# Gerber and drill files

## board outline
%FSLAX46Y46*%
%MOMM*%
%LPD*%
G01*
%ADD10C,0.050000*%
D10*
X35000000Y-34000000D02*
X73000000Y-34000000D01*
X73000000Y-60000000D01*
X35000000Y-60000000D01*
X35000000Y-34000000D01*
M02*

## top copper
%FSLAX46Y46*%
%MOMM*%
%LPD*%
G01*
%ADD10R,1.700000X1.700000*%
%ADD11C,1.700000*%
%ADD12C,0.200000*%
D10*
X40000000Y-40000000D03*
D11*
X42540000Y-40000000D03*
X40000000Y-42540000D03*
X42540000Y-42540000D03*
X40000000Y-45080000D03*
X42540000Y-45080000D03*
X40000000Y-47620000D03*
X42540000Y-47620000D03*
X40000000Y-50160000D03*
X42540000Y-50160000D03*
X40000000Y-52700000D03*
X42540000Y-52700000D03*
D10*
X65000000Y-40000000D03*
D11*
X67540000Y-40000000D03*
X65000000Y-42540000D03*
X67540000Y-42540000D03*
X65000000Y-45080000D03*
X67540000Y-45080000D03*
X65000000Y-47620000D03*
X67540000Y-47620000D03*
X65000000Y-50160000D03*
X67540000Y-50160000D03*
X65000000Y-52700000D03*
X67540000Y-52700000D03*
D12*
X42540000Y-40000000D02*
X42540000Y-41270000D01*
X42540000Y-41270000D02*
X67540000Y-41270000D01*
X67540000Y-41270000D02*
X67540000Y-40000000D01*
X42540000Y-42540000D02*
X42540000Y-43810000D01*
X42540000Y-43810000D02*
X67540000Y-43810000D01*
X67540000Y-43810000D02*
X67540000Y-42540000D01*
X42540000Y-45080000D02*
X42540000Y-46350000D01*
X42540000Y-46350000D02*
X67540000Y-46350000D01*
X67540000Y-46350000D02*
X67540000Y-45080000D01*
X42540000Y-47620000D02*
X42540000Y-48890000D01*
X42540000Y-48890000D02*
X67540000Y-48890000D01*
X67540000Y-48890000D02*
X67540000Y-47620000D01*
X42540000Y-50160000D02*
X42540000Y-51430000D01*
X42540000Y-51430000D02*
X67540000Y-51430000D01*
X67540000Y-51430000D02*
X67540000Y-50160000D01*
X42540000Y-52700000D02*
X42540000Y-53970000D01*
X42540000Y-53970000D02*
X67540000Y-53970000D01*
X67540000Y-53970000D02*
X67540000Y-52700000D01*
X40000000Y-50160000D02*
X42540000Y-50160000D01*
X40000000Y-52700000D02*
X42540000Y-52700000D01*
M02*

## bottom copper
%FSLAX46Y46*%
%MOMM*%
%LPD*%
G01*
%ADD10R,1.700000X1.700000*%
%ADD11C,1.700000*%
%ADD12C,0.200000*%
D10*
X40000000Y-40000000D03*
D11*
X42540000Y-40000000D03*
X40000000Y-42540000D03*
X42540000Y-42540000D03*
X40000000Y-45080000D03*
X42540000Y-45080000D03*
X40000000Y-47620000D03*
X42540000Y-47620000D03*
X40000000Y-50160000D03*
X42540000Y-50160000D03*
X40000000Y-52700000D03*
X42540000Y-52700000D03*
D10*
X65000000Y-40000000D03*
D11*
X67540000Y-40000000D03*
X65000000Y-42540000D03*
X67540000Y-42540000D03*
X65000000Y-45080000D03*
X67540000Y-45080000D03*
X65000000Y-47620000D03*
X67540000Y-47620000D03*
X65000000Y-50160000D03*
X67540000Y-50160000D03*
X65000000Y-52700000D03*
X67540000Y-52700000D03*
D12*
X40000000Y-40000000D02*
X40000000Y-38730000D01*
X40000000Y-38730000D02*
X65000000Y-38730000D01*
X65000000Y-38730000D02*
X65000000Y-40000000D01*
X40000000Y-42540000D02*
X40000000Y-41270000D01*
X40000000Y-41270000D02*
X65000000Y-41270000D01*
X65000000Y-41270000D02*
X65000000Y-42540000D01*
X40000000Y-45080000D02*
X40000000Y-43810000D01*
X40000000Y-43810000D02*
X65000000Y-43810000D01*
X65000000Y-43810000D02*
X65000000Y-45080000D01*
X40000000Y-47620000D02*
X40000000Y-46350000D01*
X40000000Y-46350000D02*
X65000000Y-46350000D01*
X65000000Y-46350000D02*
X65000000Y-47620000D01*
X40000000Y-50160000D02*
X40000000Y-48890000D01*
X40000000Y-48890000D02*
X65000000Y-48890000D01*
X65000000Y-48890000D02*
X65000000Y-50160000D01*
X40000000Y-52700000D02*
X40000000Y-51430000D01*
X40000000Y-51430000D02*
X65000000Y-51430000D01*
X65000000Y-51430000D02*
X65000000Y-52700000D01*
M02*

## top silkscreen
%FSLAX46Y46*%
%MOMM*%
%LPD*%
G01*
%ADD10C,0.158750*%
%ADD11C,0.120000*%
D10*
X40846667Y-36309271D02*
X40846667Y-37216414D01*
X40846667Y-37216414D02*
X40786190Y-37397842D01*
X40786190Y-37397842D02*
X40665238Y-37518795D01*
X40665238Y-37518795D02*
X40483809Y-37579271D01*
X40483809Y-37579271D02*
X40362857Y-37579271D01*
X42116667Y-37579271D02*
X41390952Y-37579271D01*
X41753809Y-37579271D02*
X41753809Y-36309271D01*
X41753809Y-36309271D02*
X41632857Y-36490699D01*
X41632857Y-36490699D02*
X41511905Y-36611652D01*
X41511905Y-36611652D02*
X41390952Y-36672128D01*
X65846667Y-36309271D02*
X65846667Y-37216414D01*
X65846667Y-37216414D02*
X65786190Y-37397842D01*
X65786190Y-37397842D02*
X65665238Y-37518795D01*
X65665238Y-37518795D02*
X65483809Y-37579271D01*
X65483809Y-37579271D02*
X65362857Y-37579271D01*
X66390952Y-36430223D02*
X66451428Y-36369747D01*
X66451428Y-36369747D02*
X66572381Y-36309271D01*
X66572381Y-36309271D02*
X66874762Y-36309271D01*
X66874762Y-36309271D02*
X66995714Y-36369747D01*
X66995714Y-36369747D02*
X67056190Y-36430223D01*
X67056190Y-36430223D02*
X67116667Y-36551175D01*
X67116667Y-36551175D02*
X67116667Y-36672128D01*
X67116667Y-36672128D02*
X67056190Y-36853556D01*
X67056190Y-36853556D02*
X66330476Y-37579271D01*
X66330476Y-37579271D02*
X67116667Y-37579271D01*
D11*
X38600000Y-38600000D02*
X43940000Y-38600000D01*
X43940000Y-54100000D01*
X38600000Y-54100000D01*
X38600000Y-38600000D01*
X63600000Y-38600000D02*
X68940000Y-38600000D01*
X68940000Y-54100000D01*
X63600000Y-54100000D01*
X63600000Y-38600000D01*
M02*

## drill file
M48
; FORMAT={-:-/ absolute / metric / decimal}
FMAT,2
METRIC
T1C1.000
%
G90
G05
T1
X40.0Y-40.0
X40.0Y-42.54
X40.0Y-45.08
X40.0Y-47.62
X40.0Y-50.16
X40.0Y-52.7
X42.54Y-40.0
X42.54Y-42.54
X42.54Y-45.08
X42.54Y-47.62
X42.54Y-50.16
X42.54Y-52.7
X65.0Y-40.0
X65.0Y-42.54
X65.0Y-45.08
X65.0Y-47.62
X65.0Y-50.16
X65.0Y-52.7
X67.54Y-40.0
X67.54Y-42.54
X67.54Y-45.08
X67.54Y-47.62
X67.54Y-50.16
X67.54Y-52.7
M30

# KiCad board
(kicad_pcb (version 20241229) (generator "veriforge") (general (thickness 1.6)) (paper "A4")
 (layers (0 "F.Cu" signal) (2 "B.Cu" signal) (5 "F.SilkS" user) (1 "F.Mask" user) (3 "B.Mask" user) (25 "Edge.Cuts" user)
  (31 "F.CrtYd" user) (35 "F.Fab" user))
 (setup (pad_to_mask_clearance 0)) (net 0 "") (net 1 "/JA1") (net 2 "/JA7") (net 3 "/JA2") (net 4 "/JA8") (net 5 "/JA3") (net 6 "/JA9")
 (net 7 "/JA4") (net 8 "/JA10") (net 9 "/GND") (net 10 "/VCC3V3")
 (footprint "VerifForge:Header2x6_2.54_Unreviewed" (layer "F.Cu") (at 40 40)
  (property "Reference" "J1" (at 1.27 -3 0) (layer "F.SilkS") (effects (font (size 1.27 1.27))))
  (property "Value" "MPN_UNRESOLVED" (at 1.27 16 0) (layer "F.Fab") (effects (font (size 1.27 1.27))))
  (fp_rect (start -1.4 -1.4) (end 3.94 14.1) (stroke (width 0.12) (type default)) (fill none) (layer "F.SilkS"))
  (pad "1" thru_hole rect (at 0 0.0) (size 1.7 1.7) (drill 1) (layers "*.Cu" "*.Mask") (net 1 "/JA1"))
  (pad "2" thru_hole circle (at 2.54 0.0) (size 1.7 1.7) (drill 1) (layers "*.Cu" "*.Mask") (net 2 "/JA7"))
  (pad "3" thru_hole circle (at 0 2.54) (size 1.7 1.7) (drill 1) (layers "*.Cu" "*.Mask") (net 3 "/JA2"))
  (pad "4" thru_hole circle (at 2.54 2.54) (size 1.7 1.7) (drill 1) (layers "*.Cu" "*.Mask") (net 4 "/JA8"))
  (pad "5" thru_hole circle (at 0 5.08) (size 1.7 1.7) (drill 1) (layers "*.Cu" "*.Mask") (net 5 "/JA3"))
  (pad "6" thru_hole circle (at 2.54 5.08) (size 1.7 1.7) (drill 1) (layers "*.Cu" "*.Mask") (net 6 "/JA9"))
  (pad "7" thru_hole circle (at 0 7.62) (size 1.7 1.7) (drill 1) (layers "*.Cu" "*.Mask") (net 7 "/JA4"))
  (pad "8" thru_hole circle (at 2.54 7.62) (size 1.7 1.7) (drill 1) (layers "*.Cu" "*.Mask") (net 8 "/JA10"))
  (pad "9" thru_hole circle (at 0 10.16) (size 1.7 1.7) (drill 1) (layers "*.Cu" "*.Mask") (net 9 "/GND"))
  (pad "10" thru_hole circle (at 2.54 10.16) (size 1.7 1.7) (drill 1) (layers "*.Cu" "*.Mask") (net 9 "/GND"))
  (pad "11" thru_hole circle (at 0 12.7) (size 1.7 1.7) (drill 1) (layers "*.Cu" "*.Mask") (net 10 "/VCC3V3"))
  (pad "12" thru_hole circle (at 2.54 12.7) (size 1.7 1.7) (drill 1) (layers "*.Cu" "*.Mask") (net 10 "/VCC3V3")))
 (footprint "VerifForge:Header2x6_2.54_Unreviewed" (layer "F.Cu") (at 65 40)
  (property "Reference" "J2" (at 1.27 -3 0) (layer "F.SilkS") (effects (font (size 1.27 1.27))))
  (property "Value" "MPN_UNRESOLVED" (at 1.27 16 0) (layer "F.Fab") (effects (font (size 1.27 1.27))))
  (fp_rect (start -1.4 -1.4) (end 3.94 14.1) (stroke (width 0.12) (type default)) (fill none) (layer "F.SilkS"))
  (pad "1" thru_hole rect (at 0 0.0) (size 1.7 1.7) (drill 1) (layers "*.Cu" "*.Mask") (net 1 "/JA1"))
  (pad "2" thru_hole circle (at 2.54 0.0) (size 1.7 1.7) (drill 1) (layers "*.Cu" "*.Mask") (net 2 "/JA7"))
  (pad "3" thru_hole circle (at 0 2.54) (size 1.7 1.7) (drill 1) (layers "*.Cu" "*.Mask") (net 3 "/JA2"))
  (pad "4" thru_hole circle (at 2.54 2.54) (size 1.7 1.7) (drill 1) (layers "*.Cu" "*.Mask") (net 4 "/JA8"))
  (pad "5" thru_hole circle (at 0 5.08) (size 1.7 1.7) (drill 1) (layers "*.Cu" "*.Mask") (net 5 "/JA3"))
  (pad "6" thru_hole circle (at 2.54 5.08) (size 1.7 1.7) (drill 1) (layers "*.Cu" "*.Mask") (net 6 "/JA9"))
  (pad "7" thru_hole circle (at 0 7.62) (size 1.7 1.7) (drill 1) (layers "*.Cu" "*.Mask") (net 7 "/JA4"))
  (pad "8" thru_hole circle (at 2.54 7.62) (size 1.7 1.7) (drill 1) (layers "*.Cu" "*.Mask") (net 8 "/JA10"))
  (pad "9" thru_hole circle (at 0 10.16) (size 1.7 1.7) (drill 1) (layers "*.Cu" "*.Mask") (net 9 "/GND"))
  (pad "10" thru_hole circle (at 2.54 10.16) (size 1.7 1.7) (drill 1) (layers "*.Cu" "*.Mask") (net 9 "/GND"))
  (pad "11" thru_hole circle (at 0 12.7) (size 1.7 1.7) (drill 1) (layers "*.Cu" "*.Mask") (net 10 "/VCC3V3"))
  (pad "12" thru_hole circle (at 2.54 12.7) (size 1.7 1.7) (drill 1) (layers "*.Cu" "*.Mask") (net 10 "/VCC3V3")))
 (gr_rect (start 35 34) (end 73 60) (stroke (width 0.05) (type default)) (fill none) (layer "Edge.Cuts"))
 (segment (start 40 40.0) (end 40 38.73) (width 0.2) (layer "B.Cu") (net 1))
 (segment (start 40 38.73) (end 65 38.73) (width 0.2) (layer "B.Cu") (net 1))
 (segment (start 65 38.73) (end 65 40.0) (width 0.2) (layer "B.Cu") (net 1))
 (segment (start 42.54 40.0) (end 42.54 41.27) (width 0.2) (layer "F.Cu") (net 2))
 (segment (start 42.54 41.27) (end 67.54 41.27) (width 0.2) (layer "F.Cu") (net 2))
 (segment (start 67.54 41.27) (end 67.54 40.0) (width 0.2) (layer "F.Cu") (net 2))
 (segment (start 40 42.54) (end 40 41.269999999999996) (width 0.2) (layer "B.Cu") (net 3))
 (segment (start 40 41.269999999999996) (end 65 41.269999999999996) (width 0.2) (layer "B.Cu") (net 3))
 (segment (start 65 41.269999999999996) (end 65 42.54) (width 0.2) (layer "B.Cu") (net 3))
 (segment (start 42.54 42.54) (end 42.54 43.81) (width 0.2) (layer "F.Cu") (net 4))
 (segment (start 42.54 43.81) (end 67.54 43.81) (width 0.2) (layer "F.Cu") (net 4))
 (segment (start 67.54 43.81) (end 67.54 42.54) (width 0.2) (layer "F.Cu") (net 4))
 (segment (start 40 45.08) (end 40 43.809999999999995) (width 0.2) (layer "B.Cu") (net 5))
 (segment (start 40 43.809999999999995) (end 65 43.809999999999995) (width 0.2) (layer "B.Cu") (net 5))
 (segment (start 65 43.809999999999995) (end 65 45.08) (width 0.2) (layer "B.Cu") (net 5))
 (segment (start 42.54 45.08) (end 42.54 46.35) (width 0.2) (layer "F.Cu") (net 6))
 (segment (start 42.54 46.35) (end 67.54 46.35) (width 0.2) (layer "F.Cu") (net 6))
 (segment (start 67.54 46.35) (end 67.54 45.08) (width 0.2) (layer "F.Cu") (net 6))
 (segment (start 40 47.62) (end 40 46.349999999999994) (width 0.2) (layer "B.Cu") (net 7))
 (segment (start 40 46.349999999999994) (end 65 46.349999999999994) (width 0.2) (layer "B.Cu") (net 7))
 (segment (start 65 46.349999999999994) (end 65 47.62) (width 0.2) (layer "B.Cu") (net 7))
 (segment (start 42.54 47.62) (end 42.54 48.89) (width 0.2) (layer "F.Cu") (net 8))
 (segment (start 42.54 48.89) (end 67.54 48.89) (width 0.2) (layer "F.Cu") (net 8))
 (segment (start 67.54 48.89) (end 67.54 47.62) (width 0.2) (layer "F.Cu") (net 8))
 (segment (start 40 50.16) (end 40 48.88999999999999) (width 0.2) (layer "B.Cu") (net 9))
 (segment (start 40 48.88999999999999) (end 65 48.88999999999999) (width 0.2) (layer "B.Cu") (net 9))
 (segment (start 65 48.88999999999999) (end 65 50.16) (width 0.2) (layer "B.Cu") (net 9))
 (segment (start 42.54 50.16) (end 42.54 51.43) (width 0.2) (layer "F.Cu") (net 9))
 (segment (start 42.54 51.43) (end 67.54 51.43) (width 0.2) (layer "F.Cu") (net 9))
 (segment (start 67.54 51.43) (end 67.54 50.16) (width 0.2) (layer "F.Cu") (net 9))
 (segment (start 40 52.7) (end 40 51.43) (width 0.2) (layer "B.Cu") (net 10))
 (segment (start 40 51.43) (end 65 51.43) (width 0.2) (layer "B.Cu") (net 10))
 (segment (start 65 51.43) (end 65 52.7) (width 0.2) (layer "B.Cu") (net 10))
 (segment (start 42.54 52.7) (end 42.54 53.970000000000006) (width 0.2) (layer "F.Cu") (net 10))
 (segment (start 42.54 53.970000000000006) (end 67.54 53.970000000000006) (width 0.2) (layer "F.Cu") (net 10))
 (segment (start 67.54 53.970000000000006) (end 67.54 52.7) (width 0.2) (layer "F.Cu") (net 10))
 (segment (start 40 50.16) (end 42.54 50.16) (width 0.2) (layer "F.Cu") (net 9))
 (segment (start 40 52.7) (end 42.54 52.7) (width 0.2) (layer "F.Cu") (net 10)))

